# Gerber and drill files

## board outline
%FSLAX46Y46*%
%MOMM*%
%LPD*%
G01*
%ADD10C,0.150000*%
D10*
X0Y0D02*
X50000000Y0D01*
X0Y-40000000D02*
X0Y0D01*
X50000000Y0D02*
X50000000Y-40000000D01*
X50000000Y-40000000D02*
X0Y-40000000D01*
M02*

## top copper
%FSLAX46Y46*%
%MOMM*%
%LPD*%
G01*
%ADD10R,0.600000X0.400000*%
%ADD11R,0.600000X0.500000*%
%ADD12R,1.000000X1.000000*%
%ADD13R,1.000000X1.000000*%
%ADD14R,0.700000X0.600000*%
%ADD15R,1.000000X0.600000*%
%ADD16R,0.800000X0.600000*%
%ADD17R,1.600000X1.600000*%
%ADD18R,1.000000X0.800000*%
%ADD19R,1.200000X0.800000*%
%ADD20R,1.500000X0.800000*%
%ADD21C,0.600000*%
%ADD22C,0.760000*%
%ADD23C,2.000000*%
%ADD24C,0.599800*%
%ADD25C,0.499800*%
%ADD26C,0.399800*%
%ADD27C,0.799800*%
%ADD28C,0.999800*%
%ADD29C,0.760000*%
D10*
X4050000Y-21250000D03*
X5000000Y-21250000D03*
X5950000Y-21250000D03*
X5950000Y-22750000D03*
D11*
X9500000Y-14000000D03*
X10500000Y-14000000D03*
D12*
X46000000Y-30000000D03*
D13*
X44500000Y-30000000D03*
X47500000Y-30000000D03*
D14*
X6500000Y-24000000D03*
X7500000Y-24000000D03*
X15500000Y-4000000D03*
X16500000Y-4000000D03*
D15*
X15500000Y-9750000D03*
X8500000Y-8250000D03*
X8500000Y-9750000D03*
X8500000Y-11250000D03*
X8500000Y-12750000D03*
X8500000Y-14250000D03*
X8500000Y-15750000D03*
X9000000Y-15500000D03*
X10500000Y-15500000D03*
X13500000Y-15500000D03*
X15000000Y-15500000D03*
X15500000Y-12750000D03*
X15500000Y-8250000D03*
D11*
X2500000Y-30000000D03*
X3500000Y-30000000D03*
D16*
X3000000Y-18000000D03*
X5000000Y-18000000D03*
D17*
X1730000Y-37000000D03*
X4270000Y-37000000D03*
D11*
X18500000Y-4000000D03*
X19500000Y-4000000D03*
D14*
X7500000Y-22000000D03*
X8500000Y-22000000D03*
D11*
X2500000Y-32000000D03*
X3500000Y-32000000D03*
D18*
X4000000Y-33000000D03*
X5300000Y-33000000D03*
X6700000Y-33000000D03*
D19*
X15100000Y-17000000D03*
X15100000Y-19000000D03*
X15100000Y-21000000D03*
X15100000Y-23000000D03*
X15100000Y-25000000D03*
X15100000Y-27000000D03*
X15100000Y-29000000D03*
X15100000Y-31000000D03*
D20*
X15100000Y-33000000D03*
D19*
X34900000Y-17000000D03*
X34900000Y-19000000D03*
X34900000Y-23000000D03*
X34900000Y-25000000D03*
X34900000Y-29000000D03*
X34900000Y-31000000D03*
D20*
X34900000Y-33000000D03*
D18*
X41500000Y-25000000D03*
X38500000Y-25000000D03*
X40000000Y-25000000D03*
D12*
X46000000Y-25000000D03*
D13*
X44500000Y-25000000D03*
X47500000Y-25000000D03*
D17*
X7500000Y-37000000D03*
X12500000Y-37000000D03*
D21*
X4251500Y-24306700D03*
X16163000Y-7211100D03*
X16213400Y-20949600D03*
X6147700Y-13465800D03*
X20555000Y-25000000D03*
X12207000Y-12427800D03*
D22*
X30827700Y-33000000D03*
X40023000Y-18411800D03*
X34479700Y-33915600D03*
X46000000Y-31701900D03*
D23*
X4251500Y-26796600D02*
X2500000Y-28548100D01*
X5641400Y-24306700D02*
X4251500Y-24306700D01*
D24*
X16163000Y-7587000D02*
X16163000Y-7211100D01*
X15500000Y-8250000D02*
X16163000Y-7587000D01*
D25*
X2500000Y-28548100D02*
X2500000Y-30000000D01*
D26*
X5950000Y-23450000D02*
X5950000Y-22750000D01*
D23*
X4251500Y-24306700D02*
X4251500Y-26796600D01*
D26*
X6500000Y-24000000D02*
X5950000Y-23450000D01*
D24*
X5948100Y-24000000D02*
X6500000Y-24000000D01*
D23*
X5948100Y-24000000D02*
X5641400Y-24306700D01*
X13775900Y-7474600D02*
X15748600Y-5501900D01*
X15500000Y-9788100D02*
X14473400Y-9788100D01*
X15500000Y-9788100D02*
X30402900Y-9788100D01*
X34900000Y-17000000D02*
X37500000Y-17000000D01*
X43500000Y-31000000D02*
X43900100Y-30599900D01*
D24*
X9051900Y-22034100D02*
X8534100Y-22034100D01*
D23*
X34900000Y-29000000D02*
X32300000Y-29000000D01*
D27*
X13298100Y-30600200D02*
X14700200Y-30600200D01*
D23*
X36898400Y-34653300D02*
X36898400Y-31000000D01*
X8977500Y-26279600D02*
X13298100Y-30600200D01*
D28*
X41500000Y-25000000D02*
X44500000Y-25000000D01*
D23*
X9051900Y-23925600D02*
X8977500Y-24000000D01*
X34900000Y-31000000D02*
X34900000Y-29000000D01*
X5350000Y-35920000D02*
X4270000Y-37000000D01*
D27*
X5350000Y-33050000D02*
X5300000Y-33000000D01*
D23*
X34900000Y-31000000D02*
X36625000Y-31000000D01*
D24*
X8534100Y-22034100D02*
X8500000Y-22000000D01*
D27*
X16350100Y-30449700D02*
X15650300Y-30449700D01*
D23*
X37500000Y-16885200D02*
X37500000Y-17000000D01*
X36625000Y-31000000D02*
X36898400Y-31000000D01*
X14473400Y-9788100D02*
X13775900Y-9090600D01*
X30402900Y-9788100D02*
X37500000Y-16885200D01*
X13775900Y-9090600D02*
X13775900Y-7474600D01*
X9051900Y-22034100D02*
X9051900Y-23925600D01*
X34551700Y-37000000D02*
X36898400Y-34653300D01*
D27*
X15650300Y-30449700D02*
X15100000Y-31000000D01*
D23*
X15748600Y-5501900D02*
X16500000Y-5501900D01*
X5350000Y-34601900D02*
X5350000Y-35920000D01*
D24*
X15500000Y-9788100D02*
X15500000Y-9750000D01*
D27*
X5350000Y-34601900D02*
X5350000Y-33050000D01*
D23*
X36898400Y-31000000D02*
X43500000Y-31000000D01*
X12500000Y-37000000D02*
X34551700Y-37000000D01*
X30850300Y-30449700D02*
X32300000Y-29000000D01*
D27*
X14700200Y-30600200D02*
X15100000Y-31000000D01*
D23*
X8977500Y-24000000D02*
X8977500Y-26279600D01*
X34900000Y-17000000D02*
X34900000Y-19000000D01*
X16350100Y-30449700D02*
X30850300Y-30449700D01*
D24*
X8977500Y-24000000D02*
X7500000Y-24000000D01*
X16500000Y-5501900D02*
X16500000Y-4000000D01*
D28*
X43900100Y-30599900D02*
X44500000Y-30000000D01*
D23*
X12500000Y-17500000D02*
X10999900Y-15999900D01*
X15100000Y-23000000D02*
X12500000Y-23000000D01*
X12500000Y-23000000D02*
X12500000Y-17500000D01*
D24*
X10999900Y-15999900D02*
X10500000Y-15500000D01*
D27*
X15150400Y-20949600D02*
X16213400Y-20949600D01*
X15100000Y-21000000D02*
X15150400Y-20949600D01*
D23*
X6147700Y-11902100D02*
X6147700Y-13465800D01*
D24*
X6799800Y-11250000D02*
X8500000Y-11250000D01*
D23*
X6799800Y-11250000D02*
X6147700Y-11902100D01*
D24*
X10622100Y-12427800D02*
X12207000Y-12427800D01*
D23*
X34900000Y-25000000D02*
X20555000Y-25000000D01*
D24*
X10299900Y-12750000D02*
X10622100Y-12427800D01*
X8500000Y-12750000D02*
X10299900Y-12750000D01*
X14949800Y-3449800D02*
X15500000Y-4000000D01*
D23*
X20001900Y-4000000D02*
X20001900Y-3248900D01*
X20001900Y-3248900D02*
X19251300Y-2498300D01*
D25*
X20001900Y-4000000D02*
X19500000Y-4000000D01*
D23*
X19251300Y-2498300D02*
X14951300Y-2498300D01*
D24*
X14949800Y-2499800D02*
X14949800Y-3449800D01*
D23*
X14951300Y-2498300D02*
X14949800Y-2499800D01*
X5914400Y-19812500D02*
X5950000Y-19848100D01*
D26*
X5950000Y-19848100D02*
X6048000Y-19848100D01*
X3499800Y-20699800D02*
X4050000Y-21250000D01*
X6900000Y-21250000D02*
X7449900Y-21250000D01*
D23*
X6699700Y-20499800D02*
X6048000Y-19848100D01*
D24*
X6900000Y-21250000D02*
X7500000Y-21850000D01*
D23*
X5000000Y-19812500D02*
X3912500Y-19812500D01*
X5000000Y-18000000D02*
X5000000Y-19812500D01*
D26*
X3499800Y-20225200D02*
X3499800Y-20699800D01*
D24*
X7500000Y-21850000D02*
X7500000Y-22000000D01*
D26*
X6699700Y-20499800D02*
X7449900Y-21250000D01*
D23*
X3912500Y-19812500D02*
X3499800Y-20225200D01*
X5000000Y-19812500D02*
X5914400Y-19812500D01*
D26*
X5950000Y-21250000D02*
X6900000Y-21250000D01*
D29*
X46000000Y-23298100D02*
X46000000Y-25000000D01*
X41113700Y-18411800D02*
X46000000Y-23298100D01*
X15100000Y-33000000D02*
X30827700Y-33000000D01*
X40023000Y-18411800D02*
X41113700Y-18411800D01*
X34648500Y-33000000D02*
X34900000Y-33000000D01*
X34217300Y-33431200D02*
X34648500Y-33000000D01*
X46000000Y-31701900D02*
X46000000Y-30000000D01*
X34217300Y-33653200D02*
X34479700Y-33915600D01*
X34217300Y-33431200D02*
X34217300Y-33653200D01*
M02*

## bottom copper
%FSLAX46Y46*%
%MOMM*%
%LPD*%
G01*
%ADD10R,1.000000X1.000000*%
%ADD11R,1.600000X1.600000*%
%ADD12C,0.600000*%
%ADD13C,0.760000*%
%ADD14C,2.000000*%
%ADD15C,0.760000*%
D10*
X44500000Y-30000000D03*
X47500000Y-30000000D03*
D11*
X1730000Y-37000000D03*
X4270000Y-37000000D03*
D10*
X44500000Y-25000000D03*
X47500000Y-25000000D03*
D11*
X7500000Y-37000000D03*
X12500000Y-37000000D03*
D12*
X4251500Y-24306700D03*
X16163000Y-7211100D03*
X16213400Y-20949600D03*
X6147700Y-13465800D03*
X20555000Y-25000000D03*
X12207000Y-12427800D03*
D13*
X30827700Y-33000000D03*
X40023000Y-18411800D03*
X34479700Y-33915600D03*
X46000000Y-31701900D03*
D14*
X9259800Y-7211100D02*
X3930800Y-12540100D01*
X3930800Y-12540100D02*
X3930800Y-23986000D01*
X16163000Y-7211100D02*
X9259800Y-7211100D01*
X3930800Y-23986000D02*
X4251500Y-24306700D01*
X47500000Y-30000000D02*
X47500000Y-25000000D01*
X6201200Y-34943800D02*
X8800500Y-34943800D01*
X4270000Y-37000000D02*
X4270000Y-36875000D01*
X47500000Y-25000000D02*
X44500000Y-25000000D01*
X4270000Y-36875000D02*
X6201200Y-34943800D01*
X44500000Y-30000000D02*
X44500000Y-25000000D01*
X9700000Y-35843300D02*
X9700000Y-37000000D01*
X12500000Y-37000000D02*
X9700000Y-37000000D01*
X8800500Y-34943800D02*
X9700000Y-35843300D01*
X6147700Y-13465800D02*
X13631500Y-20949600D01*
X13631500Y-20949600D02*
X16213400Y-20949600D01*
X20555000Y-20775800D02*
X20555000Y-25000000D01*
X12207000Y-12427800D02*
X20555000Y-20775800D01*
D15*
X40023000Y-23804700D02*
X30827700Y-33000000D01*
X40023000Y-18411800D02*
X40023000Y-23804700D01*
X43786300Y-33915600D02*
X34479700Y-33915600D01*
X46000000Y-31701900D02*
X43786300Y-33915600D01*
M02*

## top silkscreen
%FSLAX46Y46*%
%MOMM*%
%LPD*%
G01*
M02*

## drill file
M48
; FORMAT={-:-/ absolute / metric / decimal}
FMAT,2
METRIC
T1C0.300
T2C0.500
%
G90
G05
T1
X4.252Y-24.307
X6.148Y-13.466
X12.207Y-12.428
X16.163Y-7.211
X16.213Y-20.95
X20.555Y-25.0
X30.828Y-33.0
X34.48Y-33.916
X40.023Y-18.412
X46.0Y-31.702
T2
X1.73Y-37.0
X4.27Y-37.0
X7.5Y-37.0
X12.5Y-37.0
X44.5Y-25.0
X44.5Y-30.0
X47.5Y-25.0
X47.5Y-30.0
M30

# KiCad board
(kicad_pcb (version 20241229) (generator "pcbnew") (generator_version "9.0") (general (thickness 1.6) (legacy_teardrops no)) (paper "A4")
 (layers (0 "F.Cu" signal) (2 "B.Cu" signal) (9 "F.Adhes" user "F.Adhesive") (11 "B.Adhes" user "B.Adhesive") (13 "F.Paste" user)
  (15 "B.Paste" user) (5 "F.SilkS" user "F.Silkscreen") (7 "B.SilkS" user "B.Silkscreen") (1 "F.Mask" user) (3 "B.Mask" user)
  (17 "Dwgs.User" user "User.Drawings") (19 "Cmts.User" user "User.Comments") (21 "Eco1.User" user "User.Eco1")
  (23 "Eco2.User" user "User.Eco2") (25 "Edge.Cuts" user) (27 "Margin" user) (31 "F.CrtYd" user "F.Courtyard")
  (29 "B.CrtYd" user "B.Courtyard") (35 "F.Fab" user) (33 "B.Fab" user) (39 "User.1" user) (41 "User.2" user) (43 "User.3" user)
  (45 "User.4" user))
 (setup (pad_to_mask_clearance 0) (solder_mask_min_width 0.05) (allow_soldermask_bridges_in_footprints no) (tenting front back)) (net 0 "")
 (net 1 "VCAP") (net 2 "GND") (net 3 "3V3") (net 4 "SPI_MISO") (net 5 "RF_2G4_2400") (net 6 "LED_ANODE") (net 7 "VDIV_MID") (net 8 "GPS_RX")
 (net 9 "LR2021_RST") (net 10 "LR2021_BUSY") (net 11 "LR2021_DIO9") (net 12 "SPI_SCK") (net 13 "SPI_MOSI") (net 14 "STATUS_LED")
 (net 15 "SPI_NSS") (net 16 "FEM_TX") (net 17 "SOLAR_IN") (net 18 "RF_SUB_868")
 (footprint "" (layer "F.Cu") (at 5 22)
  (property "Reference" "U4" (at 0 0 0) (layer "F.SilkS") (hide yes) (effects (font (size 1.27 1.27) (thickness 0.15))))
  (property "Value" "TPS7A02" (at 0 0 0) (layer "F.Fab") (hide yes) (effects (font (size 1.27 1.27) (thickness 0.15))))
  (pad "1" smd rect (at -0.95 -0.75) (size 0.6 0.4) (layers "F.Cu" "F.Mask") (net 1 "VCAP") (thermal_bridge_angle 45))
  (pad "2" smd rect (at 0 -0.75) (size 0.6 0.4) (layers "F.Cu" "F.Mask") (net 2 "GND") (thermal_bridge_angle 45))
  (pad "3" smd rect (at 0.95 -0.75) (size 0.6 0.4) (layers "F.Cu" "F.Mask") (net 1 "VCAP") (thermal_bridge_angle 45))
  (pad "4" smd rect (at 0.95 0.75) (size 0.6 0.4) (layers "F.Cu" "F.Mask") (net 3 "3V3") (thermal_bridge_angle 45)))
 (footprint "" (layer "F.Cu") (at 10 14)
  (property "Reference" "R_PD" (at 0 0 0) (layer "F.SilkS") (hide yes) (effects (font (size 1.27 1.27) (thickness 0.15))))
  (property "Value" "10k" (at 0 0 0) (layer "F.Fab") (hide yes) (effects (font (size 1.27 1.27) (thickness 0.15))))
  (pad "1" smd rect (at -0.5 0) (size 0.6 0.5) (layers "F.Cu" "F.Mask") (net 2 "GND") (thermal_bridge_angle 45))
  (pad "2" smd rect (at 0.5 0) (size 0.6 0.5) (layers "F.Cu" "F.Mask") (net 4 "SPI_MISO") (thermal_bridge_angle 45)))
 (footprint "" (layer "F.Cu") (at 46 30)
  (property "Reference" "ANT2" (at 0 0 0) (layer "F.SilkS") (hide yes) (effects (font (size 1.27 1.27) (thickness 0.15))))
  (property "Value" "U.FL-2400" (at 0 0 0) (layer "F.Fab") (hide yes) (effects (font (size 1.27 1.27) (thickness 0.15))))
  (pad "1" smd rect (at 0 0) (size 1 1) (layers "F.Cu" "F.Mask") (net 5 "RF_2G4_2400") (thermal_bridge_angle 45))
  (pad "2" thru_hole rect (at -1.5 0) (size 1 1) (drill 0.5) (layers "*.Cu" "*.Mask") (remove_unused_layers no) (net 2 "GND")
   (thermal_bridge_angle 45))
  (pad "3" thru_hole rect (at 1.5 0) (size 1 1) (drill 0.5) (layers "*.Cu" "*.Mask") (remove_unused_layers no) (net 2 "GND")
   (thermal_bridge_angle 45)))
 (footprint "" (layer "F.Cu") (at 7 24)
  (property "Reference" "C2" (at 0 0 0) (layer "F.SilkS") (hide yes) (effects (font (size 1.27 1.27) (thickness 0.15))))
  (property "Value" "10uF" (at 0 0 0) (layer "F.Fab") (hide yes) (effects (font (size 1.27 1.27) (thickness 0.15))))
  (pad "1" smd rect (at -0.5 0) (size 0.7 0.6) (layers "F.Cu" "F.Mask") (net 3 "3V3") (thermal_bridge_angle 45))
  (pad "2" smd rect (at 0.5 0) (size 0.7 0.6) (layers "F.Cu" "F.Mask") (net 2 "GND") (thermal_bridge_angle 45)))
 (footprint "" (layer "F.Cu") (at 16 4)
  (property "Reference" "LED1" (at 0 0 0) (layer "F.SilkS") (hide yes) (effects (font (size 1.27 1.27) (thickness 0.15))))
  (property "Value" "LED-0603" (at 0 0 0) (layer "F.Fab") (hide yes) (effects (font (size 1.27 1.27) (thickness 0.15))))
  (pad "A" smd rect (at -0.5 0) (size 0.7 0.6) (layers "F.Cu" "F.Mask") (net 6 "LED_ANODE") (thermal_bridge_angle 45))
  (pad "K" smd rect (at 0.5 0) (size 0.7 0.6) (layers "F.Cu" "F.Mask") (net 2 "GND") (thermal_bridge_angle 45)))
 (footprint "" (layer "F.Cu") (at 12 12)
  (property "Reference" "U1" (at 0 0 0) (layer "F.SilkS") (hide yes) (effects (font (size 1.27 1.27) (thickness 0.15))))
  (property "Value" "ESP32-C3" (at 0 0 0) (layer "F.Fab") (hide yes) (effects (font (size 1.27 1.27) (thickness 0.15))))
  (pad "GND" smd rect (at 3.5 -2.25) (size 1 0.6) (layers "F.Cu" "F.Mask") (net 2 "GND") (thermal_bridge_angle 45))
  (pad "GPIO0" smd rect (at -3.5 -3.75) (size 1 0.6) (layers "F.Cu" "F.Mask") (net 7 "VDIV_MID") (thermal_bridge_angle 45))
  (pad "GPIO1" smd rect (at -3.5 -2.25) (size 1 0.6) (layers "F.Cu" "F.Mask") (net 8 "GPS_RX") (thermal_bridge_angle 45))
  (pad "GPIO2" smd rect (at -3.5 -0.75) (size 1 0.6) (layers "F.Cu" "F.Mask") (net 4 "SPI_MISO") (thermal_bridge_angle 45))
  (pad "GPIO3" smd rect (at -3.5 0.75) (size 1 0.6) (layers "F.Cu" "F.Mask") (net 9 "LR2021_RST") (thermal_bridge_angle 45))
  (pad "GPIO4" smd rect (at -3.5 2.25) (size 1 0.6) (layers "F.Cu" "F.Mask") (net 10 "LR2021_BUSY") (thermal_bridge_angle 45))
  (pad "GPIO5" smd rect (at -3.5 3.75) (size 1 0.6) (layers "F.Cu" "F.Mask") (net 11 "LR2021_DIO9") (thermal_bridge_angle 45))
  (pad "GPIO6" smd rect (at -3 3.5) (size 1 0.6) (layers "F.Cu" "F.Mask") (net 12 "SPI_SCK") (thermal_bridge_angle 45))
  (pad "GPIO7" smd rect (at -1.5 3.5) (size 1 0.6) (layers "F.Cu" "F.Mask") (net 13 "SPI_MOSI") (thermal_bridge_angle 45))
  (pad "GPIO9" smd rect (at 1.5 3.5) (size 1 0.6) (layers "F.Cu" "F.Mask") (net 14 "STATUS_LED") (thermal_bridge_angle 45))
  (pad "GPIO10" smd rect (at 3 3.5) (size 1 0.6) (layers "F.Cu" "F.Mask") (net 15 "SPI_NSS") (thermal_bridge_angle 45))
  (pad "GPIO19" smd rect (at 3.5 0.75) (size 1 0.6) (layers "F.Cu" "F.Mask") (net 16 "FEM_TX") (thermal_bridge_angle 45))
  (pad "VCC" smd rect (at 3.5 -3.75) (size 1 0.6) (layers "F.Cu" "F.Mask") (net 3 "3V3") (thermal_bridge_angle 45)))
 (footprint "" (layer "F.Cu") (at 3 30)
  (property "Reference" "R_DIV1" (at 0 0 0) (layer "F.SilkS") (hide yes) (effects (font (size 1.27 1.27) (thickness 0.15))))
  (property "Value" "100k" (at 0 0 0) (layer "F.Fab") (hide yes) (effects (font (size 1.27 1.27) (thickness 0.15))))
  (pad "1" smd rect (at -0.5 0) (size 0.6 0.5) (layers "F.Cu" "F.Mask") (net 3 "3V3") (thermal_bridge_angle 45))
  (pad "2" smd rect (at 0.5 0) (size 0.6 0.5) (layers "F.Cu" "F.Mask") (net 7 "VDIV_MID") (thermal_bridge_angle 45)))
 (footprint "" (layer "F.Cu") (at 4 18)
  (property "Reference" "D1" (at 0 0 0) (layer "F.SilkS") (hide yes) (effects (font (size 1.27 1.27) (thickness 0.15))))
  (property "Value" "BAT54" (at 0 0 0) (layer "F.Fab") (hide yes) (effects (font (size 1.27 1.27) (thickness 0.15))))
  (pad "A" smd rect (at -1 0) (size 0.8 0.6) (layers "F.Cu" "F.Mask") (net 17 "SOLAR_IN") (thermal_bridge_angle 45))
  (pad "K" smd rect (at 1 0) (size 0.8 0.6) (layers "F.Cu" "F.Mask") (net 1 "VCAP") (thermal_bridge_angle 45)))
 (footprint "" (layer "F.Cu") (at 3 37)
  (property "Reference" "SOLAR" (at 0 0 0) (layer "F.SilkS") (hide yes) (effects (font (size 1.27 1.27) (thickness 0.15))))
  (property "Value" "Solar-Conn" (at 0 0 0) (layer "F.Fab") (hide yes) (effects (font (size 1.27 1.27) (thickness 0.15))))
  (pad "1" thru_hole rect (at -1.27 0) (size 1.6 1.6) (drill 0.5) (layers "*.Cu" "*.Mask") (remove_unused_layers no) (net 17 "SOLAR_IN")
   (thermal_bridge_angle 45))
  (pad "2" thru_hole rect (at 1.27 0) (size 1.6 1.6) (drill 0.5) (layers "*.Cu" "*.Mask") (remove_unused_layers no) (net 2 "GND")
   (thermal_bridge_angle 45)))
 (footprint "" (layer "F.Cu") (at 19 4)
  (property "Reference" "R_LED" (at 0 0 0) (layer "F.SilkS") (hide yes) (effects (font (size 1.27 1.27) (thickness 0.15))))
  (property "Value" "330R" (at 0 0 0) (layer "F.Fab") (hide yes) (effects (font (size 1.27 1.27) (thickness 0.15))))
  (pad "1" smd rect (at -0.5 0) (size 0.6 0.5) (layers "F.Cu" "F.Mask") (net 14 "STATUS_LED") (thermal_bridge_angle 45))
  (pad "2" smd rect (at 0.5 0) (size 0.6 0.5) (layers "F.Cu" "F.Mask") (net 6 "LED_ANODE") (thermal_bridge_angle 45)))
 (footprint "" (layer "F.Cu") (at 8 22)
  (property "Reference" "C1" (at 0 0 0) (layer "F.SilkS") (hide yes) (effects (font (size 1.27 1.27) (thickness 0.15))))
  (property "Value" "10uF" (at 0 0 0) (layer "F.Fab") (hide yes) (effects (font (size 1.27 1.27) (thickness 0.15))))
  (pad "1" smd rect (at -0.5 0) (size 0.7 0.6) (layers "F.Cu" "F.Mask") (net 1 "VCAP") (thermal_bridge_angle 45))
  (pad "2" smd rect (at 0.5 0) (size 0.7 0.6) (layers "F.Cu" "F.Mask") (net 2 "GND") (thermal_bridge_angle 45)))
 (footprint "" (layer "F.Cu") (at 3 32)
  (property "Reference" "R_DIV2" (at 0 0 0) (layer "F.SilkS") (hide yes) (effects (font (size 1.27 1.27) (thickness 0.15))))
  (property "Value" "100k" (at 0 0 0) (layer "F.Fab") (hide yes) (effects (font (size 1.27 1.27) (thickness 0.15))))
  (pad "1" smd rect (at -0.5 0) (size 0.6 0.5) (layers "F.Cu" "F.Mask") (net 7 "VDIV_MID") (thermal_bridge_angle 45))
  (pad "2" smd rect (at 0.5 0) (size 0.6 0.5) (layers "F.Cu" "F.Mask") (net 2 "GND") (thermal_bridge_angle 45)))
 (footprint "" (layer "F.Cu") (at 6 33)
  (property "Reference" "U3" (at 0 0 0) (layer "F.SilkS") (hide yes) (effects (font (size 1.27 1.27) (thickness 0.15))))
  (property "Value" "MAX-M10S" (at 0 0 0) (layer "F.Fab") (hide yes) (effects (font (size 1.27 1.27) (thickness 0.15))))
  (pad "1" smd rect (at -2 0) (size 1 0.8) (layers "F.Cu" "F.Mask") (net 3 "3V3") (thermal_bridge_angle 45))
  (pad "2" smd rect (at -0.7 0) (size 1 0.8) (layers "F.Cu" "F.Mask") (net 2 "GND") (thermal_bridge_angle 45))
  (pad "3" smd rect (at 0.7 0) (size 1 0.8) (layers "F.Cu" "F.Mask") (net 8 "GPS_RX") (thermal_bridge_angle 45)))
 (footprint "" (layer "F.Cu") (at 25 25)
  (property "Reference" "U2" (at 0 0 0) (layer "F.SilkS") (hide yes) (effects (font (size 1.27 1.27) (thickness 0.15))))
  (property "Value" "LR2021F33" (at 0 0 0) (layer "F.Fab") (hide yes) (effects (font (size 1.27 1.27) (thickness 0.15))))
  (pad "1" smd rect (at -9.9 -8) (size 1.2 0.8) (layers "F.Cu" "F.Mask") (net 3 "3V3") (thermal_bridge_angle 45))
  (pad "2" smd rect (at -9.9 -6) (size 1.2 0.8) (layers "F.Cu" "F.Mask") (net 2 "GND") (thermal_bridge_angle 45))
  (pad "3" smd rect (at -9.9 -4) (size 1.2 0.8) (layers "F.Cu" "F.Mask") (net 4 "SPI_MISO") (thermal_bridge_angle 45))
  (pad "4" smd rect (at -9.9 -2) (size 1.2 0.8) (layers "F.Cu" "F.Mask") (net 13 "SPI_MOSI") (thermal_bridge_angle 45))
  (pad "5" smd rect (at -9.9 0) (size 1.2 0.8) (layers "F.Cu" "F.Mask") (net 12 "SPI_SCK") (thermal_bridge_angle 45))
  (pad "6" smd rect (at -9.9 2) (size 1.2 0.8) (layers "F.Cu" "F.Mask") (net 15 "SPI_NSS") (thermal_bridge_angle 45))
  (pad "7" smd rect (at -9.9 4) (size 1.2 0.8) (layers "F.Cu" "F.Mask") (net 10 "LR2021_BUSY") (thermal_bridge_angle 45))
  (pad "8" smd rect (at -9.9 6) (size 1.2 0.8) (layers "F.Cu" "F.Mask") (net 2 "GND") (thermal_bridge_angle 45))
  (pad "9" smd rect (at -9.9 8) (size 1.5 0.8) (layers "F.Cu" "F.Mask") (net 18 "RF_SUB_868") (thermal_bridge_angle 45))
  (pad "10" smd rect (at 9.9 -8) (size 1.2 0.8) (layers "F.Cu" "F.Mask") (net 2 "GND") (thermal_bridge_angle 45))
  (pad "11" smd rect (at 9.9 -6) (size 1.2 0.8) (layers "F.Cu" "F.Mask") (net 2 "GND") (thermal_bridge_angle 45))
  (pad "13" smd rect (at 9.9 -2) (size 1.2 0.8) (layers "F.Cu" "F.Mask") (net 11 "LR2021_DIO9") (thermal_bridge_angle 45))
  (pad "14" smd rect (at 9.9 0) (size 1.2 0.8) (layers "F.Cu" "F.Mask") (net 9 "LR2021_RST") (thermal_bridge_angle 45))
  (pad "16" smd rect (at 9.9 4) (size 1.2 0.8) (layers "F.Cu" "F.Mask") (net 2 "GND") (thermal_bridge_angle 45))
  (pad "17" smd rect (at 9.9 6) (size 1.2 0.8) (layers "F.Cu" "F.Mask") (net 2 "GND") (thermal_bridge_angle 45))
  (pad "18" smd rect (at 9.9 8) (size 1.5 0.8) (layers "F.Cu" "F.Mask") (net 5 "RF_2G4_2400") (thermal_bridge_angle 45)))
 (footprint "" (layer "F.Cu") (at 40 25)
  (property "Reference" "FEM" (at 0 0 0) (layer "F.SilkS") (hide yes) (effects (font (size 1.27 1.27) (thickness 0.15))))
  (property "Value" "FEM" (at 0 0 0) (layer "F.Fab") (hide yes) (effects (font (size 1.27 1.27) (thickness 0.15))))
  (pad "GND" smd rect (at 1.5 0) (size 1 0.8) (layers "F.Cu" "F.Mask") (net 2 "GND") (thermal_bridge_angle 45))
  (pad "TX" smd rect (at -1.5 0) (size 1 0.8) (layers "F.Cu" "F.Mask") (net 16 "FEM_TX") (thermal_bridge_angle 45))
  (pad "VCC" smd rect (at 0 0) (size 1 0.8) (layers "F.Cu" "F.Mask") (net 3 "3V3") (thermal_bridge_angle 45)))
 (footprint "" (layer "F.Cu") (at 46 25)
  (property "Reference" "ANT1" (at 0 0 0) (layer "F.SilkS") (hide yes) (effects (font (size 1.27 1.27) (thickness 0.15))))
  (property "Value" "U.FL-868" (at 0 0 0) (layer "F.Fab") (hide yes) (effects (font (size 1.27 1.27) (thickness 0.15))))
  (pad "1" smd rect (at 0 0) (size 1 1) (layers "F.Cu" "F.Mask") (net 18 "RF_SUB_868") (thermal_bridge_angle 45))
  (pad "2" thru_hole rect (at -1.5 0) (size 1 1) (drill 0.5) (layers "*.Cu" "*.Mask") (remove_unused_layers no) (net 2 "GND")
   (thermal_bridge_angle 45))
  (pad "3" thru_hole rect (at 1.5 0) (size 1 1) (drill 0.5) (layers "*.Cu" "*.Mask") (remove_unused_layers no) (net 2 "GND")
   (thermal_bridge_angle 45)))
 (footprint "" (layer "F.Cu") (at 10 37)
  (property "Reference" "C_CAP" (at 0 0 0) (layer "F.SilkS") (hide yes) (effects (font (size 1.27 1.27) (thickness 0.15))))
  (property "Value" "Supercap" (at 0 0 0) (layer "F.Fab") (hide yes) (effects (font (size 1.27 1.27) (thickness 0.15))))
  (pad "1" thru_hole rect (at -2.5 0) (size 1.6 1.6) (drill 0.5) (layers "*.Cu" "*.Mask") (remove_unused_layers no) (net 1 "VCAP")
   (thermal_bridge_angle 45))
  (pad "2" thru_hole rect (at 2.5 0) (size 1.6 1.6) (drill 0.5) (layers "*.Cu" "*.Mask") (remove_unused_layers no) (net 2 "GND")
   (thermal_bridge_angle 45)))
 (gr_line (start 0 0) (end 50 0) (stroke (width 0.15) (type default)) (layer "Edge.Cuts"))
 (gr_line (start 0 40) (end 0 0) (stroke (width 0.15) (type default)) (layer "Edge.Cuts"))
 (gr_line (start 50 0) (end 50 40) (stroke (width 0.15) (type default)) (layer "Edge.Cuts"))
 (gr_line (start 50 40) (end 0 40) (stroke (width 0.15) (type default)) (layer "Edge.Cuts"))
 (segment (start 4.2515 26.7966) (end 2.5 28.5481) (width 2) (layer "F.Cu") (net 3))
 (segment (start 5.6414 24.3067) (end 4.2515 24.3067) (width 2) (layer "F.Cu") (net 3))
 (segment (start 16.163 7.587) (end 16.163 7.2111) (width 0.5998) (layer "F.Cu") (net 3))
 (segment (start 15.5 8.25) (end 16.163 7.587) (width 0.5998) (layer "F.Cu") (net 3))
 (segment (start 2.5 28.5481) (end 2.5 30) (width 0.4998) (layer "F.Cu") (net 3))
 (segment (start 5.95 23.45) (end 5.95 22.75) (width 0.3998) (layer "F.Cu") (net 3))
 (segment (start 4.2515 24.3067) (end 4.2515 26.7966) (width 2) (layer "F.Cu") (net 3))
 (segment (start 6.5 24) (end 5.95 23.45) (width 0.3998) (layer "F.Cu") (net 3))
 (segment (start 5.9481 24) (end 6.5 24) (width 0.5998) (layer "F.Cu") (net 3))
 (segment (start 5.9481 24) (end 5.6414 24.3067) (width 2) (layer "F.Cu") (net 3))
 (via (at 4.2515 24.3067) (size 0.6) (drill 0.3) (layers "F.Cu" "B.Cu") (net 3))
 (via (at 16.163 7.2111) (size 0.6) (drill 0.3) (layers "F.Cu" "B.Cu") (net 3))
 (segment (start 9.2598 7.2111) (end 3.9308 12.5401) (width 2) (layer "B.Cu") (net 3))
 (segment (start 3.9308 12.5401) (end 3.9308 23.986) (width 2) (layer "B.Cu") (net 3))
 (segment (start 16.163 7.2111) (end 9.2598 7.2111) (width 2) (layer "B.Cu") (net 3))
 (segment (start 3.9308 23.986) (end 4.2515 24.3067) (width 2) (layer "B.Cu") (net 3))
 (segment (start 13.7759 7.4746) (end 15.7486 5.5019) (width 2) (layer "F.Cu") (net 2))
 (segment (start 15.5 9.7881) (end 14.4734 9.7881) (width 2) (layer "F.Cu") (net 2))
 (segment (start 15.5 9.7881) (end 30.4029 9.7881) (width 2) (layer "F.Cu") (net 2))
 (segment (start 34.9 17) (end 37.5 17) (width 2) (layer "F.Cu") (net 2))
 (segment (start 43.5 31) (end 43.9001 30.5999) (width 2) (layer "F.Cu") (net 2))
 (segment (start 9.0519 22.0341) (end 8.5341 22.0341) (width 0.5998) (layer "F.Cu") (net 2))
 (segment (start 34.9 29) (end 32.3 29) (width 2) (layer "F.Cu") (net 2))
 (segment (start 13.2981 30.6002) (end 14.7002 30.6002) (width 0.7998) (layer "F.Cu") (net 2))
 (segment (start 36.8984 34.6533) (end 36.8984 31) (width 2) (layer "F.Cu") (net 2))
 (segment (start 8.9775 26.2796) (end 13.2981 30.6002) (width 2) (layer "F.Cu") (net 2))
 (segment (start 41.5 25) (end 44.5 25) (width 0.9998) (layer "F.Cu") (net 2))
 (segment (start 9.0519 23.9256) (end 8.9775 24) (width 2) (layer "F.Cu") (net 2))
 (segment (start 34.9 31) (end 34.9 29) (width 2) (layer "F.Cu") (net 2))
 (segment (start 5.35 35.92) (end 4.27 37) (width 2) (layer "F.Cu") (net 2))
 (segment (start 5.35 33.05) (end 5.3 33) (width 0.7998) (layer "F.Cu") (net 2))
 (segment (start 34.9 31) (end 36.625 31) (width 2) (layer "F.Cu") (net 2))
 (segment (start 8.5341 22.0341) (end 8.5 22) (width 0.5998) (layer "F.Cu") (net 2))
 (segment (start 16.3501 30.4497) (end 15.6503 30.4497) (width 0.7998) (layer "F.Cu") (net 2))
 (segment (start 37.5 16.8852) (end 37.5 17) (width 2) (layer "F.Cu") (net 2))
 (segment (start 36.625 31) (end 36.8984 31) (width 2) (layer "F.Cu") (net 2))
 (segment (start 14.4734 9.7881) (end 13.7759 9.0906) (width 2) (layer "F.Cu") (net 2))
 (segment (start 30.4029 9.7881) (end 37.5 16.8852) (width 2) (layer "F.Cu") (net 2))
 (segment (start 13.7759 9.0906) (end 13.7759 7.4746) (width 2) (layer "F.Cu") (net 2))
 (segment (start 9.0519 22.0341) (end 9.0519 23.9256) (width 2) (layer "F.Cu") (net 2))
 (segment (start 34.5517 37) (end 36.8984 34.6533) (width 2) (layer "F.Cu") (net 2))
 (segment (start 15.6503 30.4497) (end 15.1 31) (width 0.7998) (layer "F.Cu") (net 2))
 (segment (start 15.7486 5.5019) (end 16.5 5.5019) (width 2) (layer "F.Cu") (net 2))
 (segment (start 5.35 34.6019) (end 5.35 35.92) (width 2) (layer "F.Cu") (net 2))
 (segment (start 15.5 9.7881) (end 15.5 9.75) (width 0.5998) (layer "F.Cu") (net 2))
 (segment (start 5.35 34.6019) (end 5.35 33.05) (width 0.7998) (layer "F.Cu") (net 2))
 (segment (start 36.8984 31) (end 43.5 31) (width 2) (layer "F.Cu") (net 2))
 (segment (start 12.5 37) (end 34.5517 37) (width 2) (layer "F.Cu") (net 2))
 (segment (start 30.8503 30.4497) (end 32.3 29) (width 2) (layer "F.Cu") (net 2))
 (segment (start 14.7002 30.6002) (end 15.1 31) (width 0.7998) (layer "F.Cu") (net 2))
 (segment (start 8.9775 24) (end 8.9775 26.2796) (width 2) (layer "F.Cu") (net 2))
 (segment (start 34.9 17) (end 34.9 19) (width 2) (layer "F.Cu") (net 2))
 (segment (start 16.3501 30.4497) (end 30.8503 30.4497) (width 2) (layer "F.Cu") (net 2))
 (segment (start 8.9775 24) (end 7.5 24) (width 0.5998) (layer "F.Cu") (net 2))
 (segment (start 16.5 5.5019) (end 16.5 4) (width 0.5998) (layer "F.Cu") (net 2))
 (segment (start 43.9001 30.5999) (end 44.5 30) (width 0.9998) (layer "F.Cu") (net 2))
 (segment (start 47.5 30) (end 47.5 25) (width 2) (layer "B.Cu") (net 2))
 (segment (start 6.2012 34.9438) (end 8.8005 34.9438) (width 2) (layer "B.Cu") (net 2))
 (segment (start 4.27 37) (end 4.27 36.875) (width 2) (layer "B.Cu") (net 2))
 (segment (start 47.5 25) (end 44.5 25) (width 2) (layer "B.Cu") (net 2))
 (segment (start 4.27 36.875) (end 6.2012 34.9438) (width 2) (layer "B.Cu") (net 2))
 (segment (start 44.5 30) (end 44.5 25) (width 2) (layer "B.Cu") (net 2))
 (segment (start 9.7 35.8433) (end 9.7 37) (width 2) (layer "B.Cu") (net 2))
 (segment (start 12.5 37) (end 9.7 37) (width 2) (layer "B.Cu") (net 2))
 (segment (start 8.8005 34.9438) (end 9.7 35.8433) (width 2) (layer "B.Cu") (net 2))
 (segment (start 12.5 17.5) (end 10.9999 15.9999) (width 2) (layer "F.Cu") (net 13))
 (segment (start 15.1 23) (end 12.5 23) (width 2) (layer "F.Cu") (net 13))
 (segment (start 12.5 23) (end 12.5 17.5) (width 2) (layer "F.Cu") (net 13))
 (segment (start 10.9999 15.9999) (end 10.5 15.5) (width 0.5998) (layer "F.Cu") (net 13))
 (segment (start 15.1504 20.9496) (end 16.2134 20.9496) (width 0.7998) (layer "F.Cu") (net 4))
 (segment (start 15.1 21) (end 15.1504 20.9496) (width 0.7998) (layer "F.Cu") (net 4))
 (segment (start 6.1477 11.9021) (end 6.1477 13.4658) (width 2) (layer "F.Cu") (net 4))
 (segment (start 6.7998 11.25) (end 8.5 11.25) (width 0.5998) (layer "F.Cu") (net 4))
 (segment (start 6.7998 11.25) (end 6.1477 11.9021) (width 2) (layer "F.Cu") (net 4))
 (via (at 16.2134 20.9496) (size 0.6) (drill 0.3) (layers "F.Cu" "B.Cu") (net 4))
 (via (at 6.1477 13.4658) (size 0.6) (drill 0.3) (layers "F.Cu" "B.Cu") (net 4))
 (segment (start 6.1477 13.4658) (end 13.6315 20.9496) (width 2) (layer "B.Cu") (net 4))
 (segment (start 13.6315 20.9496) (end 16.2134 20.9496) (width 2) (layer "B.Cu") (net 4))
 (segment (start 10.6221 12.4278) (end 12.207 12.4278) (width 0.5998) (layer "F.Cu") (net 9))
 (segment (start 34.9 25) (end 20.555 25) (width 2) (layer "F.Cu") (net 9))
 (segment (start 10.2999 12.75) (end 10.6221 12.4278) (width 0.5998) (layer "F.Cu") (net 9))
 (segment (start 8.5 12.75) (end 10.2999 12.75) (width 0.5998) (layer "F.Cu") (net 9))
 (via (at 20.555 25) (size 0.6) (drill 0.3) (layers "F.Cu" "B.Cu") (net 9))
 (via (at 12.207 12.4278) (size 0.6) (drill 0.3) (layers "F.Cu" "B.Cu") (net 9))
 (segment (start 20.555 20.7758) (end 20.555 25) (width 2) (layer "B.Cu") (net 9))
 (segment (start 12.207 12.4278) (end 20.555 20.7758) (width 2) (layer "B.Cu") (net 9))
 (segment (start 14.9498 3.4498) (end 15.5 4) (width 0.5998) (layer "F.Cu") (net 6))
 (segment (start 20.0019 4) (end 20.0019 3.2489) (width 2) (layer "F.Cu") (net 6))
 (segment (start 20.0019 3.2489) (end 19.2513 2.4983) (width 2) (layer "F.Cu") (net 6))
 (segment (start 20.0019 4) (end 19.5 4) (width 0.4998) (layer "F.Cu") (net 6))
 (segment (start 19.2513 2.4983) (end 14.9513 2.4983) (width 2) (layer "F.Cu") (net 6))
 (segment (start 14.9498 2.4998) (end 14.9498 3.4498) (width 0.5998) (layer "F.Cu") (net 6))
 (segment (start 14.9513 2.4983) (end 14.9498 2.4998) (width 2) (layer "F.Cu") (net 6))
 (segment (start 5.9144 19.8125) (end 5.95 19.8481) (width 2) (layer "F.Cu") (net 1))
 (segment (start 5.95 19.8481) (end 6.048 19.8481) (width 0.3998) (layer "F.Cu") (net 1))
 (segment (start 3.4998 20.6998) (end 4.05 21.25) (width 0.3998) (layer "F.Cu") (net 1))
 (segment (start 6.9 21.25) (end 7.4499 21.25) (width 0.3998) (layer "F.Cu") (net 1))
 (segment (start 6.6997 20.4998) (end 6.048 19.8481) (width 2) (layer "F.Cu") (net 1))
 (segment (start 6.9 21.25) (end 7.5 21.85) (width 0.5998) (layer "F.Cu") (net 1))
 (segment (start 5 19.8125) (end 3.9125 19.8125) (width 2) (layer "F.Cu") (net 1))
 (segment (start 5 18) (end 5 19.8125) (width 2) (layer "F.Cu") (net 1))
 (segment (start 3.4998 20.2252) (end 3.4998 20.6998) (width 0.3998) (layer "F.Cu") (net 1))
 (segment (start 7.5 21.85) (end 7.5 22) (width 0.5998) (layer "F.Cu") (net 1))
 (segment (start 6.6997 20.4998) (end 7.4499 21.25) (width 0.3998) (layer "F.Cu") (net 1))
 (segment (start 3.9125 19.8125) (end 3.4998 20.2252) (width 2) (layer "F.Cu") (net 1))
 (segment (start 5 19.8125) (end 5.9144 19.8125) (width 2) (layer "F.Cu") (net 1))
 (segment (start 5.95 21.25) (end 6.9 21.25) (width 0.3998) (layer "F.Cu") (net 1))
 (segment (start 46 23.2981) (end 46 25) (width 0.76) (layer "F.Cu") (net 18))
 (segment (start 41.1137 18.4118) (end 46 23.2981) (width 0.76) (layer "F.Cu") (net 18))
 (segment (start 15.1 33) (end 30.8277 33) (width 0.76) (layer "F.Cu") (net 18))
 (segment (start 40.023 18.4118) (end 41.1137 18.4118) (width 0.76) (layer "F.Cu") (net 18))
 (via (at 30.8277 33) (size 0.76) (drill 0.3) (layers "F.Cu" "B.Cu") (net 18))
 (via (at 40.023 18.4118) (size 0.76) (drill 0.3) (layers "F.Cu" "B.Cu") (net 18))
 (segment (start 40.023 23.8047) (end 30.8277 33) (width 0.76) (layer "B.Cu") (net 18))
 (segment (start 40.023 18.4118) (end 40.023 23.8047) (width 0.76) (layer "B.Cu") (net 18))
 (segment (start 34.6485 33) (end 34.9 33) (width 0.76) (layer "F.Cu") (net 5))
 (segment (start 34.2173 33.4312) (end 34.6485 33) (width 0.76) (layer "F.Cu") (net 5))
 (segment (start 46 31.7019) (end 46 30) (width 0.76) (layer "F.Cu") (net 5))
 (segment (start 34.2173 33.6532) (end 34.4797 33.9156) (width 0.76) (layer "F.Cu") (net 5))
 (segment (start 34.2173 33.4312) (end 34.2173 33.6532) (width 0.76) (layer "F.Cu") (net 5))
 (via (at 34.4797 33.9156) (size 0.76) (drill 0.3) (layers "F.Cu" "B.Cu") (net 5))
 (via (at 46 31.7019) (size 0.76) (drill 0.3) (layers "F.Cu" "B.Cu") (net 5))
 (segment (start 43.7863 33.9156) (end 34.4797 33.9156) (width 0.76) (layer "B.Cu") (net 5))
 (segment (start 46 31.7019) (end 43.7863 33.9156) (width 0.76) (layer "B.Cu") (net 5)))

